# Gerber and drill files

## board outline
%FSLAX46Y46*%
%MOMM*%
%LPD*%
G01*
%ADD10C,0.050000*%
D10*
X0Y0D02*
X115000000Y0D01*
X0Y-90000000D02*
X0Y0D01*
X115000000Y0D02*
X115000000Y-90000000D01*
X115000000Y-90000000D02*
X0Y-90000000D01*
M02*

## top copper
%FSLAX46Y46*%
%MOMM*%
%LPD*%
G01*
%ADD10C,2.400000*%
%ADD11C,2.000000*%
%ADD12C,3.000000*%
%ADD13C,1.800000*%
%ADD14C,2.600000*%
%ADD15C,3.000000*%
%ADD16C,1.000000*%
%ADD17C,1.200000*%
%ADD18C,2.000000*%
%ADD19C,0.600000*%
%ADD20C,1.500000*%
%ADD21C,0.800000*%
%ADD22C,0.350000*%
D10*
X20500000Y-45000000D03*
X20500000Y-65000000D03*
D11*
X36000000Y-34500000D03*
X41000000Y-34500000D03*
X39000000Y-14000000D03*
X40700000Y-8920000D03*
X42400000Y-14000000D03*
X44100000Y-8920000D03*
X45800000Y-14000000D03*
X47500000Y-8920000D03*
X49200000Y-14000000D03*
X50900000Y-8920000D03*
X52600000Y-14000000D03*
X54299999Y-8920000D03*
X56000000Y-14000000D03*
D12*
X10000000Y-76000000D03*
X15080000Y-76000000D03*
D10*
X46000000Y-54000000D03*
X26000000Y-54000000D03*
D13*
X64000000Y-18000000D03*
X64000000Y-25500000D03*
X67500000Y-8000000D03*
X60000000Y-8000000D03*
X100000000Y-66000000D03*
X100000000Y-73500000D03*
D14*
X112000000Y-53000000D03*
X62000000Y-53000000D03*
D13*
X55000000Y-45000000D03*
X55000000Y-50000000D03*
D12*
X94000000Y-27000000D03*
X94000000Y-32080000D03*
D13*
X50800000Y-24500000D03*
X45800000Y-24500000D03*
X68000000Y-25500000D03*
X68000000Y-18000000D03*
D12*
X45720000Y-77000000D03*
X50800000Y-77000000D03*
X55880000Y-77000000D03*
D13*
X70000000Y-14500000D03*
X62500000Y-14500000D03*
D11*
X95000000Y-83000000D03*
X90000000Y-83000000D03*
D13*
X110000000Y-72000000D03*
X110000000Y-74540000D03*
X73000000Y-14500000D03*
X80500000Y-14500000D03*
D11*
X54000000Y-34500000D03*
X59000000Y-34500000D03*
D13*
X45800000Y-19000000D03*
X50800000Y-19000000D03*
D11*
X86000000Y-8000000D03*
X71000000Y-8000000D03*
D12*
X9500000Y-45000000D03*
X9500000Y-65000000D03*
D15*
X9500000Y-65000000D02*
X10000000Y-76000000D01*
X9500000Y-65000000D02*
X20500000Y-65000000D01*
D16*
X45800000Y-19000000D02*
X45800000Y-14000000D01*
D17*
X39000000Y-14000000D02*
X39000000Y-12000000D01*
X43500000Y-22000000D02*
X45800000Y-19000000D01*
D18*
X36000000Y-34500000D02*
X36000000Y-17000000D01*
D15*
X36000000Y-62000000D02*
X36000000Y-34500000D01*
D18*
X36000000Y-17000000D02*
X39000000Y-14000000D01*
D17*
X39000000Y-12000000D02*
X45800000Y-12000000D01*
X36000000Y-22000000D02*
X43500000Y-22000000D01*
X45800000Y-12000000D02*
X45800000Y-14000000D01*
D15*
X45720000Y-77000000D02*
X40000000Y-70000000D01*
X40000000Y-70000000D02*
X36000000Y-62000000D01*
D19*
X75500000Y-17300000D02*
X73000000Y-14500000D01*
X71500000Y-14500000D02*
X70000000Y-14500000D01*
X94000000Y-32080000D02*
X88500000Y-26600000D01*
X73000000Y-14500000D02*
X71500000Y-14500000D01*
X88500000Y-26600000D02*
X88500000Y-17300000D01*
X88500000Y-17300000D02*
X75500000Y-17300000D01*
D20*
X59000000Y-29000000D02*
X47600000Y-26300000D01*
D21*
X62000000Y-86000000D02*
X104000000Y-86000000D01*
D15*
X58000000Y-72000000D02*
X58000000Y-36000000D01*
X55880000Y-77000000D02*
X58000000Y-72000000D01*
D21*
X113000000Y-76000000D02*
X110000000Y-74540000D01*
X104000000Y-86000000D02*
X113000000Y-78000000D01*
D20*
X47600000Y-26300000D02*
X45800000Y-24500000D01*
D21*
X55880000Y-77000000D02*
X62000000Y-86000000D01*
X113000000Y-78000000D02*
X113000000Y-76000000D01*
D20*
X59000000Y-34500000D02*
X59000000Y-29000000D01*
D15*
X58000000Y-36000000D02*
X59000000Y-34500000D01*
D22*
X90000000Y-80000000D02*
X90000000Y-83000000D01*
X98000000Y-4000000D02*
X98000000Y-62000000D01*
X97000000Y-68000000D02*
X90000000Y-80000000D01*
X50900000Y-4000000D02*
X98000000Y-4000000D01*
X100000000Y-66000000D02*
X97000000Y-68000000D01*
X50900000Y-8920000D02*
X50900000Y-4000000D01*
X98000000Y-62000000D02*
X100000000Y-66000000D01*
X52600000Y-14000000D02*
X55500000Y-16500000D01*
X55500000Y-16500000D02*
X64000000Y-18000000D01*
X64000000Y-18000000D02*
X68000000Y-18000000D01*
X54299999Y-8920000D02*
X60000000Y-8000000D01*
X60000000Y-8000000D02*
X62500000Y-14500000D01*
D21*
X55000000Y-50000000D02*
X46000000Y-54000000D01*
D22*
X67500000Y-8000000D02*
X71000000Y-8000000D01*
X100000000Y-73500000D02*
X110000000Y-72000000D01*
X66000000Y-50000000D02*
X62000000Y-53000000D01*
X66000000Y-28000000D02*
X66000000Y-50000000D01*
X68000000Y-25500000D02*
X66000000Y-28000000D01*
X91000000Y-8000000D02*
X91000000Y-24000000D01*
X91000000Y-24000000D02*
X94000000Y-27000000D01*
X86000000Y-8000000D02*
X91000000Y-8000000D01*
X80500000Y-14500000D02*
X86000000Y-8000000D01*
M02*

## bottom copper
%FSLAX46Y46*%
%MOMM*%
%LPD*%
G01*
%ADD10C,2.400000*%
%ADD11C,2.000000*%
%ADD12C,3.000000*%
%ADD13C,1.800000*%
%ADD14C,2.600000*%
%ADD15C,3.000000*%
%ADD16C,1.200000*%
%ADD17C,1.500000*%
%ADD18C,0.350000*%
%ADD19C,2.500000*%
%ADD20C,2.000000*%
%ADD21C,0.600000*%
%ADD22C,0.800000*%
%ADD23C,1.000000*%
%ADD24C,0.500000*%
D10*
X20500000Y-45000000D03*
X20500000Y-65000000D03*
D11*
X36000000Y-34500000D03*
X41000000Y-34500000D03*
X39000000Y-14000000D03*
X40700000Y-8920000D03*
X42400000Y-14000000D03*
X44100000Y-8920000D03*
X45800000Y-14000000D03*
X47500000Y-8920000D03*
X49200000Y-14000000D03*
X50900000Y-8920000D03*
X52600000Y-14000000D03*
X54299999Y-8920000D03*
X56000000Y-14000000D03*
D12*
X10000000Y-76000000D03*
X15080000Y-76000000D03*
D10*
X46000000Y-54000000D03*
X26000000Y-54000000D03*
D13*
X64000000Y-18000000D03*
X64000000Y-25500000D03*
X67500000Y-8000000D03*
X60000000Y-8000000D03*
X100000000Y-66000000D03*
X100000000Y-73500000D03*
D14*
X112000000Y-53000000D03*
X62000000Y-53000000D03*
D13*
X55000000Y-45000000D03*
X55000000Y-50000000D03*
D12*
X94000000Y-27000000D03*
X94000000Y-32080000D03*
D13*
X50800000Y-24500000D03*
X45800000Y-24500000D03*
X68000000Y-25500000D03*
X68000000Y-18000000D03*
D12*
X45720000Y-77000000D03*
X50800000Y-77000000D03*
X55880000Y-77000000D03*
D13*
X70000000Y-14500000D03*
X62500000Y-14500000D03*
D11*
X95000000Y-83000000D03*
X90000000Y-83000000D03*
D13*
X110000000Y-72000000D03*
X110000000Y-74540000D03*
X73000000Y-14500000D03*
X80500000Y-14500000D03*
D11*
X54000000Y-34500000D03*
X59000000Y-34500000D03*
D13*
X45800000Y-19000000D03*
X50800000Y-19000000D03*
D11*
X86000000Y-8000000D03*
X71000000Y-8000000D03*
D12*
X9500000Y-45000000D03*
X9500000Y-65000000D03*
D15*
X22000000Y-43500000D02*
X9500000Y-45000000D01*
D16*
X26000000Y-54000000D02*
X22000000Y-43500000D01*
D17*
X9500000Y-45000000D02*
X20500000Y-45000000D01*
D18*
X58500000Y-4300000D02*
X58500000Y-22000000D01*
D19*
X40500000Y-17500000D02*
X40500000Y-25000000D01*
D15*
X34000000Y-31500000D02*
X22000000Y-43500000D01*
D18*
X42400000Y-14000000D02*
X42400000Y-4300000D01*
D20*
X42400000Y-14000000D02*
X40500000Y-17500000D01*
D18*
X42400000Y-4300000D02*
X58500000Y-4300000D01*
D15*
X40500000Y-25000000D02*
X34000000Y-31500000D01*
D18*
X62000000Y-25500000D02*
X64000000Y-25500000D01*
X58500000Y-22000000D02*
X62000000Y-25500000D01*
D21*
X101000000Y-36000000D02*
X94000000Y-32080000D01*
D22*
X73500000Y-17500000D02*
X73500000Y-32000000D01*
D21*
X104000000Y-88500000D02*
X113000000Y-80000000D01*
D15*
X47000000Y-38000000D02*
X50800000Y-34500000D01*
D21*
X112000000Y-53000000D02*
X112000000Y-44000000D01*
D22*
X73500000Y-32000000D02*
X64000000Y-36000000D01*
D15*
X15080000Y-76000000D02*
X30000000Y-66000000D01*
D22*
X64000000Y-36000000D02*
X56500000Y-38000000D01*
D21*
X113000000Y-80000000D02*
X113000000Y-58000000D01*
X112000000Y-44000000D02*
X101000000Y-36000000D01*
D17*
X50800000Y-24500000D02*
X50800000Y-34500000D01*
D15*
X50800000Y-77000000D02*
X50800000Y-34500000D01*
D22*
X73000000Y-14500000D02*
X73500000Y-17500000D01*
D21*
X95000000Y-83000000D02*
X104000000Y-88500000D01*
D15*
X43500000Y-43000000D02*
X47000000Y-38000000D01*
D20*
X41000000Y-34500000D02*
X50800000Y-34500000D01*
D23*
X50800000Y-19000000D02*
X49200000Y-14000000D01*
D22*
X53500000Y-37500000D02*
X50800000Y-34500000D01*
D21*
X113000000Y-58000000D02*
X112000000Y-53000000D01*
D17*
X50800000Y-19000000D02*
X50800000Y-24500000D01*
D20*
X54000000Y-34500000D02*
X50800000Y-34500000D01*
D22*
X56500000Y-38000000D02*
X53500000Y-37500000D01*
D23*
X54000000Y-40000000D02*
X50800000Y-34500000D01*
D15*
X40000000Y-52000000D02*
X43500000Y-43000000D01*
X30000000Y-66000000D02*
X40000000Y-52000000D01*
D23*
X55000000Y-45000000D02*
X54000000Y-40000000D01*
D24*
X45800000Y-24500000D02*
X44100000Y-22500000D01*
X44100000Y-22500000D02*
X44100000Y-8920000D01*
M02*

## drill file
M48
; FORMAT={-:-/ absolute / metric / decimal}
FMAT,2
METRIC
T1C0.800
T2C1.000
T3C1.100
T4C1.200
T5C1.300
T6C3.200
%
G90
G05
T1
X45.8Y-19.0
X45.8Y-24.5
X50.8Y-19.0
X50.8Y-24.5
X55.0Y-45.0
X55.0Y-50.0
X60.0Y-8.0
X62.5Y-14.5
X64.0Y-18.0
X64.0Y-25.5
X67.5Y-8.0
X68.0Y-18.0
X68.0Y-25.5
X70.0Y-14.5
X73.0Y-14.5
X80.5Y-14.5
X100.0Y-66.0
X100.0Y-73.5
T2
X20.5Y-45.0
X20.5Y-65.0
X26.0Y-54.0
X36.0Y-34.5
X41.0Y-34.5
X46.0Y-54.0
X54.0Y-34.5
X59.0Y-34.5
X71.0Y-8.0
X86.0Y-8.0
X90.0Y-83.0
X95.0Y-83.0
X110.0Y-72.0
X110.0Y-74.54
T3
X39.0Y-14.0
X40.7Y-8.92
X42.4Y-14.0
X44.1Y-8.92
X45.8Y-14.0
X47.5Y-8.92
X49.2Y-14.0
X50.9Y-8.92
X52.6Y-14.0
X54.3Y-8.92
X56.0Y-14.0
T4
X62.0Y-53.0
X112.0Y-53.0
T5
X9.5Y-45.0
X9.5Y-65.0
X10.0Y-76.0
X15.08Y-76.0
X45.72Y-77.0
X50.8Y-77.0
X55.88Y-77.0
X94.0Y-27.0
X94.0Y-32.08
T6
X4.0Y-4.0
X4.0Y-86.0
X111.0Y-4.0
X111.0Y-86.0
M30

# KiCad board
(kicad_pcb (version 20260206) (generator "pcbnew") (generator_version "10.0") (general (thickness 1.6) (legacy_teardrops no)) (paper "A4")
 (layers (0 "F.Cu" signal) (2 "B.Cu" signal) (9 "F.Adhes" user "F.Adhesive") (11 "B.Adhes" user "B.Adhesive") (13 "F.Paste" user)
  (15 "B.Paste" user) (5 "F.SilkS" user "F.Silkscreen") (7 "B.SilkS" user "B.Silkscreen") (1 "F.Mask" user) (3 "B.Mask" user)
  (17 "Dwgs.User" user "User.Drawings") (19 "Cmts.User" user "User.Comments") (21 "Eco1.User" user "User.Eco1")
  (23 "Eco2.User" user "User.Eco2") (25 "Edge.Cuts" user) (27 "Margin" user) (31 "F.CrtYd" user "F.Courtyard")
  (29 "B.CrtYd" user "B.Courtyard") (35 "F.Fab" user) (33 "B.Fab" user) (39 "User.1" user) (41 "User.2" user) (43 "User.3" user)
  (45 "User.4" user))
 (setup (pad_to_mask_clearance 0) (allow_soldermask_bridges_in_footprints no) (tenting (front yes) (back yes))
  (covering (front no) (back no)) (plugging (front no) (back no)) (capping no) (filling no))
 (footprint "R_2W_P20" (layer "F.Cu") (at 20.5 45 -90)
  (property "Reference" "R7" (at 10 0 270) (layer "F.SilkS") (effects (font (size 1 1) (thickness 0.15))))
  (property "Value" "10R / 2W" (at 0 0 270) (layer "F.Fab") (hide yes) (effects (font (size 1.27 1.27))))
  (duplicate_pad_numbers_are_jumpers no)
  (pad "1" thru_hole circle (at 0 0 270) (size 2.4 2.4) (drill 1) (layers "*.Cu" "*.Mask") (remove_unused_layers no) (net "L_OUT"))
  (pad "2" thru_hole circle (at 20 0 270) (size 2.4 2.4) (drill 1) (layers "*.Cu" "*.Mask") (remove_unused_layers no) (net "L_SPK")))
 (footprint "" (layer "F.Cu") (at 111 4)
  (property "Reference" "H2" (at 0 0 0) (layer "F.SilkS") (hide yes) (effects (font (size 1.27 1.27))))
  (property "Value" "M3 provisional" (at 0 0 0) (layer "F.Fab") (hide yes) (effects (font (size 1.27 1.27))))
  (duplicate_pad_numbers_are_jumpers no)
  (pad "" np_thru_hole circle (at 0 0) (size 3.2 3.2) (drill 3.2) (layers "*.Cu" "*.Mask")))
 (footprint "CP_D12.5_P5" (layer "F.Cu") (at 36 34.5)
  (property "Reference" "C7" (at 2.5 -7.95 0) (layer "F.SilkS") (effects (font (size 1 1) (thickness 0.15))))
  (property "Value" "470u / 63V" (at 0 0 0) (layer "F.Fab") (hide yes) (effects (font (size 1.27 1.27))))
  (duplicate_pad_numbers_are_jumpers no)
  (pad "1" thru_hole circle (at 0 0) (size 2 2) (drill 1) (layers "*.Cu" "*.Mask") (remove_unused_layers no) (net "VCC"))
  (pad "2" thru_hole circle (at 5 0) (size 2 2) (drill 1) (layers "*.Cu" "*.Mask") (remove_unused_layers no) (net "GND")))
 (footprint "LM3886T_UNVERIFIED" (layer "F.Cu") (at 39 14)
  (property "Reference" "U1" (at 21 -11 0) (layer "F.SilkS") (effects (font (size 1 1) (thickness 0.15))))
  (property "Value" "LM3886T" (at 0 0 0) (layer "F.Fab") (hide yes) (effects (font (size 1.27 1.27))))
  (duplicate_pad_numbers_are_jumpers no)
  (pad "1" thru_hole circle (at 0 0) (size 2 2) (drill 1.1) (layers "*.Cu" "*.Mask") (remove_unused_layers no) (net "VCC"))
  (pad "2" thru_hole circle (at 1.7 -5.08) (size 2 2) (drill 1.1) (layers "*.Cu" "*.Mask") (remove_unused_layers no)
   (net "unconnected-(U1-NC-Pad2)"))
  (pad "3" thru_hole circle (at 3.4 0) (size 2 2) (drill 1.1) (layers "*.Cu" "*.Mask") (remove_unused_layers no) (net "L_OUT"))
  (pad "4" thru_hole circle (at 5.1 -5.08) (size 2 2) (drill 1.1) (layers "*.Cu" "*.Mask") (remove_unused_layers no) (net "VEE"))
  (pad "5" thru_hole circle (at 6.8 0) (size 2 2) (drill 1.1) (layers "*.Cu" "*.Mask") (remove_unused_layers no) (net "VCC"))
  (pad "6" thru_hole circle (at 8.5 -5.08) (size 2 2) (drill 1.1) (layers "*.Cu" "*.Mask") (remove_unused_layers no)
   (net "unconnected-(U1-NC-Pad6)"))
  (pad "7" thru_hole circle (at 10.2 0) (size 2 2) (drill 1.1) (layers "*.Cu" "*.Mask") (remove_unused_layers no) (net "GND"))
  (pad "8" thru_hole circle (at 11.9 -5.08) (size 2 2) (drill 1.1) (layers "*.Cu" "*.Mask") (remove_unused_layers no) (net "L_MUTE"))
  (pad "9" thru_hole circle (at 13.6 0) (size 2 2) (drill 1.1) (layers "*.Cu" "*.Mask") (remove_unused_layers no) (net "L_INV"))
  (pad "10" thru_hole circle (at 15.299999 -5.08) (size 2 2) (drill 1.1) (layers "*.Cu" "*.Mask") (remove_unused_layers no) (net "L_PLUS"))
  (pad "11" thru_hole circle (at 17 0) (size 2 2) (drill 1.1) (layers "*.Cu" "*.Mask") (remove_unused_layers no)
   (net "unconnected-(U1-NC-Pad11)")))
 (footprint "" (layer "F.Cu") (at 4 4)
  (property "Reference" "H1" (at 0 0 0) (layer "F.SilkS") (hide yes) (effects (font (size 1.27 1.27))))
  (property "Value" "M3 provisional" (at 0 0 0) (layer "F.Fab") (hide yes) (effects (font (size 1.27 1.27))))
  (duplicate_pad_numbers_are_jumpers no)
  (pad "" np_thru_hole circle (at 0 0) (size 3.2 3.2) (drill 3.2) (layers "*.Cu" "*.Mask")))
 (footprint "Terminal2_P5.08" (layer "F.Cu") (at 10 76)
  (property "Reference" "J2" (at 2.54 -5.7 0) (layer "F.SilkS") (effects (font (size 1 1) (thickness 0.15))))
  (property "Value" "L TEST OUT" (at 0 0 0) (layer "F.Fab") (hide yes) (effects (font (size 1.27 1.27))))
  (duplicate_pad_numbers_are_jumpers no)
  (pad "1" thru_hole circle (at 0 0) (size 3 3) (drill 1.3) (layers "*.Cu" "*.Mask") (remove_unused_layers no) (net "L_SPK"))
  (pad "2" thru_hole circle (at 5.08 0) (size 3 3) (drill 1.3) (layers "*.Cu" "*.Mask") (remove_unused_layers no) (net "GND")))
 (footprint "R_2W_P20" (layer "F.Cu") (at 46 54 180)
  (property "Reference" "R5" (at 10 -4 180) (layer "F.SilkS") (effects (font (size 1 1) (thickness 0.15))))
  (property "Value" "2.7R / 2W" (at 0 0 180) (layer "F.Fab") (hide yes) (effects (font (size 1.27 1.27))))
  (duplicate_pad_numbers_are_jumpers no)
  (pad "1" thru_hole circle (at 0 0 180) (size 2.4 2.4) (drill 1) (layers "*.Cu" "*.Mask") (remove_unused_layers no) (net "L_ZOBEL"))
  (pad "2" thru_hole circle (at 20 0 180) (size 2.4 2.4) (drill 1) (layers "*.Cu" "*.Mask") (remove_unused_layers no) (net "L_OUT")))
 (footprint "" (layer "F.Cu") (at 4 86)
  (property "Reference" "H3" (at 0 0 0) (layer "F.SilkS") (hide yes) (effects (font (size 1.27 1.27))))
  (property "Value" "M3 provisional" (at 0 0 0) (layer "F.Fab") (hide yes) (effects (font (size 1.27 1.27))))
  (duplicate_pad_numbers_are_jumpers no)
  (pad "" np_thru_hole circle (at 0 0) (size 3.2 3.2) (drill 3.2) (layers "*.Cu" "*.Mask")))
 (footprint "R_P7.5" (layer "F.Cu") (at 64 18 -90)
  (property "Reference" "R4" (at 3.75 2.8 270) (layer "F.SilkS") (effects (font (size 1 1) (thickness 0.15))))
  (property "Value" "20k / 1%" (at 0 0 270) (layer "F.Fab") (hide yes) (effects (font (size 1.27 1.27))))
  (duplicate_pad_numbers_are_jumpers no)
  (pad "1" thru_hole circle (at 0 0 270) (size 1.8 1.8) (drill 0.8) (layers "*.Cu" "*.Mask") (remove_unused_layers no) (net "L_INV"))
  (pad "2" thru_hole circle (at 7.5 0 270) (size 1.8 1.8) (drill 0.8) (layers "*.Cu" "*.Mask") (remove_unused_layers no) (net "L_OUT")))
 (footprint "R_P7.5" (layer "F.Cu") (at 67.5 8 180)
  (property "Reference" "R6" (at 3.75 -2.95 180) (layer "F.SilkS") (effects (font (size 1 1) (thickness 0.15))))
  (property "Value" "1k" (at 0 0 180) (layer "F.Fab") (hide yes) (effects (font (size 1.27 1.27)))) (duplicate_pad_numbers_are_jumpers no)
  (pad "1" thru_hole circle (at 0 0 180) (size 1.8 1.8) (drill 0.8) (layers "*.Cu" "*.Mask") (remove_unused_layers no) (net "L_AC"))
  (pad "2" thru_hole circle (at 7.5 0 180) (size 1.8 1.8) (drill 0.8) (layers "*.Cu" "*.Mask") (remove_unused_layers no) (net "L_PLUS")))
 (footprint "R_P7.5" (layer "F.Cu") (at 100 66 -90)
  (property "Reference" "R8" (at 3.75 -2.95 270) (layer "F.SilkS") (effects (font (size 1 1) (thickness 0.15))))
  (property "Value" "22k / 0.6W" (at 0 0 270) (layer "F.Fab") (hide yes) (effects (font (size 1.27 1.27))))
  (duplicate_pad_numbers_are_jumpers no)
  (pad "1" thru_hole circle (at 0 0 270) (size 1.8 1.8) (drill 0.8) (layers "*.Cu" "*.Mask") (remove_unused_layers no) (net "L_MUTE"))
  (pad "2" thru_hole circle (at 7.5 0 270) (size 1.8 1.8) (drill 0.8) (layers "*.Cu" "*.Mask") (remove_unused_layers no) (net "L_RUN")))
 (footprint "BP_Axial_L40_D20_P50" (layer "F.Cu") (at 112 53 180)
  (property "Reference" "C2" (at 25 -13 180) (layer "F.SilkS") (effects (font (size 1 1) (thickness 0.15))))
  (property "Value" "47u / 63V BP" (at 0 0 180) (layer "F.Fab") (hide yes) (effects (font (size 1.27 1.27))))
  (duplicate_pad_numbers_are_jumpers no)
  (pad "1" thru_hole circle (at 0 0 180) (size 2.6 2.6) (drill 1.2) (layers "*.Cu" "*.Mask") (remove_unused_layers no) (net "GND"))
  (pad "2" thru_hole circle (at 50 0 180) (size 2.6 2.6) (drill 1.2) (layers "*.Cu" "*.Mask") (remove_unused_layers no) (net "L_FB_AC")))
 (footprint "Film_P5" (layer "F.Cu") (at 55 45 -90)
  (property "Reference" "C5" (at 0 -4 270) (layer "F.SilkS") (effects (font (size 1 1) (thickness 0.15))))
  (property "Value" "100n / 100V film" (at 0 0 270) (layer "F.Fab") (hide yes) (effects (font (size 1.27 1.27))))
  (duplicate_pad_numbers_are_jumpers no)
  (pad "1" thru_hole circle (at 0 0 270) (size 1.8 1.8) (drill 0.8) (layers "*.Cu" "*.Mask") (remove_unused_layers no) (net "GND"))
  (pad "2" thru_hole circle (at 5 0 270) (size 1.8 1.8) (drill 0.8) (layers "*.Cu" "*.Mask") (remove_unused_layers no) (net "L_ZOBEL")))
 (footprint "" (layer "F.Cu") (at 111 86)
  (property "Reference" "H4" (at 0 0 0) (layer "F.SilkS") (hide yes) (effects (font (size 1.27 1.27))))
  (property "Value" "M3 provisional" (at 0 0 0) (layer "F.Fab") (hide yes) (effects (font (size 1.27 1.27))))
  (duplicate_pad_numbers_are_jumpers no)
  (pad "" np_thru_hole circle (at 0 0) (size 3.2 3.2) (drill 3.2) (layers "*.Cu" "*.Mask")))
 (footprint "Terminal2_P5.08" (layer "F.Cu") (at 94 27 -90)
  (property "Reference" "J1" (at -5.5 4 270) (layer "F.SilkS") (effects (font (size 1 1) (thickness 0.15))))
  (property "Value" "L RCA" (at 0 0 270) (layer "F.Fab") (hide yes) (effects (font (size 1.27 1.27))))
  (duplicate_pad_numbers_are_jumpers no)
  (pad "1" thru_hole circle (at 0 0 270) (size 3 3) (drill 1.3) (layers "*.Cu" "*.Mask") (remove_unused_layers no) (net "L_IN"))
  (pad "2" thru_hole circle (at 5.08 0 270) (size 3 3) (drill 1.3) (layers "*.Cu" "*.Mask") (remove_unused_layers no) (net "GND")))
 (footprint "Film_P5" (layer "F.Cu") (at 50.8 24.5 180)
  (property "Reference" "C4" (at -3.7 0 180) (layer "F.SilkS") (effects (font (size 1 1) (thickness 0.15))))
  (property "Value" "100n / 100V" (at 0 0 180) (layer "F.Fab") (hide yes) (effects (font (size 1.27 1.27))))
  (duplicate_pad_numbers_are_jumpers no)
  (pad "1" thru_hole circle (at 0 0 180) (size 1.8 1.8) (drill 0.8) (layers "*.Cu" "*.Mask") (remove_unused_layers no) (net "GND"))
  (pad "2" thru_hole circle (at 5 0 180) (size 1.8 1.8) (drill 0.8) (layers "*.Cu" "*.Mask") (remove_unused_layers no) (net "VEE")))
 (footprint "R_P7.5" (layer "F.Cu") (at 68 25.5 90)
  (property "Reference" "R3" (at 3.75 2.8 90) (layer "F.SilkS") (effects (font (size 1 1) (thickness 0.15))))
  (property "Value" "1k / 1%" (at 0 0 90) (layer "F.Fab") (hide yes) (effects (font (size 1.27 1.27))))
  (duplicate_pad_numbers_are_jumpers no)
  (pad "1" thru_hole circle (at 0 0 90) (size 1.8 1.8) (drill 0.8) (layers "*.Cu" "*.Mask") (remove_unused_layers no) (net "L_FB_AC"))
  (pad "2" thru_hole circle (at 7.5 0 90) (size 1.8 1.8) (drill 0.8) (layers "*.Cu" "*.Mask") (remove_unused_layers no) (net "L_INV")))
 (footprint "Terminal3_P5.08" (layer "F.Cu") (at 45.72 77)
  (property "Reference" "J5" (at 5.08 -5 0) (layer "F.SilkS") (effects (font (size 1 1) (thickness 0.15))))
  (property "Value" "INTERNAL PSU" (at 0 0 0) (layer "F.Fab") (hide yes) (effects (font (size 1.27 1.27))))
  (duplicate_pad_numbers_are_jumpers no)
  (pad "1" thru_hole circle (at 0 0) (size 3 3) (drill 1.3) (layers "*.Cu" "*.Mask") (remove_unused_layers no) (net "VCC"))
  (pad "2" thru_hole circle (at 5.08 0) (size 3 3) (drill 1.3) (layers "*.Cu" "*.Mask") (remove_unused_layers no) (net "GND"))
  (pad "3" thru_hole circle (at 10.16 0) (size 3 3) (drill 1.3) (layers "*.Cu" "*.Mask") (remove_unused_layers no) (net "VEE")))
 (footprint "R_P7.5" (layer "F.Cu") (at 70 14.5 180)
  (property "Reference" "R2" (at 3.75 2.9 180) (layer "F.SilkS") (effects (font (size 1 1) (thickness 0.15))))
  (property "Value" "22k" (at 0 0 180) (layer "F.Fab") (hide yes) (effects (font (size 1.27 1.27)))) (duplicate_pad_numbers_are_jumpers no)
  (pad "1" thru_hole circle (at 0 0 180) (size 1.8 1.8) (drill 0.8) (layers "*.Cu" "*.Mask") (remove_unused_layers no) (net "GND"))
  (pad "2" thru_hole circle (at 7.5 0 180) (size 1.8 1.8) (drill 0.8) (layers "*.Cu" "*.Mask") (remove_unused_layers no) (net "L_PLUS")))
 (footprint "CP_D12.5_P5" (layer "F.Cu") (at 95 83 180)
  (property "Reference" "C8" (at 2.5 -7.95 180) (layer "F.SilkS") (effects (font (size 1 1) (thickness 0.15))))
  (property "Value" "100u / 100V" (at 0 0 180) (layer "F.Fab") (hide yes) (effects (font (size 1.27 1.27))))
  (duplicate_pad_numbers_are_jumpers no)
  (pad "1" thru_hole circle (at 0 0 180) (size 2 2) (drill 1) (layers "*.Cu" "*.Mask") (remove_unused_layers no) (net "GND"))
  (pad "2" thru_hole circle (at 5 0 180) (size 2 2) (drill 1) (layers "*.Cu" "*.Mask") (remove_unused_layers no) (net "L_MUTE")))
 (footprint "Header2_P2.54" (layer "F.Cu") (at 110 72 -90)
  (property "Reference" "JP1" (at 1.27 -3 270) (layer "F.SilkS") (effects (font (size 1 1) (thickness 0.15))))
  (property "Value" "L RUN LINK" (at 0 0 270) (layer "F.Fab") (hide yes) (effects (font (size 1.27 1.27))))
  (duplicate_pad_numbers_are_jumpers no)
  (pad "1" thru_hole circle (at 0 0 270) (size 1.8 1.8) (drill 1) (layers "*.Cu" "*.Mask") (remove_unused_layers no) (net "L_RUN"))
  (pad "2" thru_hole circle (at 2.54 0 270) (size 1.8 1.8) (drill 1) (layers "*.Cu" "*.Mask") (remove_unused_layers no) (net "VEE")))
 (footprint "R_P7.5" (layer "F.Cu") (at 73 14.5)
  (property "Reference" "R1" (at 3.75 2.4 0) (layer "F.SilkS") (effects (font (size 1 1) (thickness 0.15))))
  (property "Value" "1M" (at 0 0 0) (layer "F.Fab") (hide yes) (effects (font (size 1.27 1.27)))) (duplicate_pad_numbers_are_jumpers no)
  (pad "1" thru_hole circle (at 0 0) (size 1.8 1.8) (drill 0.8) (layers "*.Cu" "*.Mask") (remove_unused_layers no) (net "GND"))
  (pad "2" thru_hole circle (at 7.5 0) (size 1.8 1.8) (drill 0.8) (layers "*.Cu" "*.Mask") (remove_unused_layers no) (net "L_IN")))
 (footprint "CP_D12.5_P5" (layer "F.Cu") (at 54 34.5)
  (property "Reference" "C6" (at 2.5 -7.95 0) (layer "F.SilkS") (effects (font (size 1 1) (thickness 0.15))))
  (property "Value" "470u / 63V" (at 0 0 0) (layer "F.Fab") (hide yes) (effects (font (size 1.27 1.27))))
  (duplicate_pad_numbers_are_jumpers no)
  (pad "1" thru_hole circle (at 0 0) (size 2 2) (drill 1) (layers "*.Cu" "*.Mask") (remove_unused_layers no) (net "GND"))
  (pad "2" thru_hole circle (at 5 0) (size 2 2) (drill 1) (layers "*.Cu" "*.Mask") (remove_unused_layers no) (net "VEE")))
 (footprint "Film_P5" (layer "F.Cu") (at 45.8 19)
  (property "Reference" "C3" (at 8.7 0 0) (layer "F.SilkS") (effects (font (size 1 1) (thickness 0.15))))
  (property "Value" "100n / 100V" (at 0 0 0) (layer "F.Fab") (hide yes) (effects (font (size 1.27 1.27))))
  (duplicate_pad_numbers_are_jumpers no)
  (pad "1" thru_hole circle (at 0 0) (size 1.8 1.8) (drill 0.8) (layers "*.Cu" "*.Mask") (remove_unused_layers no) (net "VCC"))
  (pad "2" thru_hole circle (at 5 0) (size 1.8 1.8) (drill 0.8) (layers "*.Cu" "*.Mask") (remove_unused_layers no) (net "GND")))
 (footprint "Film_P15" (layer "F.Cu") (at 86 8 180)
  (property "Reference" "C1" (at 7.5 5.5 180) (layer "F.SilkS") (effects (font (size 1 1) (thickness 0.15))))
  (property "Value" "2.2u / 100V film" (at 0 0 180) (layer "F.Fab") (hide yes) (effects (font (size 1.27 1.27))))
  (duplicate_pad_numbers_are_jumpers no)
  (pad "1" thru_hole circle (at 0 0 180) (size 2 2) (drill 1) (layers "*.Cu" "*.Mask") (remove_unused_layers no) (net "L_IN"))
  (pad "2" thru_hole circle (at 15 0 180) (size 2 2) (drill 1) (layers "*.Cu" "*.Mask") (remove_unused_layers no) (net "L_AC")))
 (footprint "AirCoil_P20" (layer "F.Cu") (at 9.5 45 -90)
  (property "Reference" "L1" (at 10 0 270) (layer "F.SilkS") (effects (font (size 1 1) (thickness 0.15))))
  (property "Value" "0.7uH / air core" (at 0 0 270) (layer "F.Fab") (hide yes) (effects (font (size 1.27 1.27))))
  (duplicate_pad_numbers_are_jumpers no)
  (pad "1" thru_hole circle (at 0 0 270) (size 3 3) (drill 1.3) (layers "*.Cu" "*.Mask") (remove_unused_layers no) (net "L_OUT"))
  (pad "2" thru_hole circle (at 20 0 270) (size 3 3) (drill 1.3) (layers "*.Cu" "*.Mask") (remove_unused_layers no) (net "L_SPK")))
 (gr_line (start 0 0) (end 115 0) (stroke (width 0.05) (type default)) (layer "Edge.Cuts"))
 (gr_line (start 0 90) (end 0 0) (stroke (width 0.05) (type default)) (layer "Edge.Cuts"))
 (gr_line (start 115 0) (end 115 90) (stroke (width 0.05) (type default)) (layer "Edge.Cuts"))
 (gr_line (start 115 90) (end 0 90) (stroke (width 0.05) (type default)) (layer "Edge.Cuts"))
 (segment (start 22 43.5) (end 9.5 45) (width 3) (layer "B.Cu") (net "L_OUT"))
 (segment (start 26 54) (end 22 43.5) (width 1.2) (layer "B.Cu") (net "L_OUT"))
 (segment (start 9.5 45) (end 20.5 45) (width 1.5) (layer "B.Cu") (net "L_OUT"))
 (segment (start 58.5 4.3) (end 58.5 22) (width 0.35) (layer "B.Cu") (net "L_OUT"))
 (segment (start 40.5 17.5) (end 40.5 25) (width 2.5) (layer "B.Cu") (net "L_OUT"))
 (segment (start 34 31.5) (end 22 43.5) (width 3) (layer "B.Cu") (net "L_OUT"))
 (segment (start 42.4 14) (end 42.4 4.3) (width 0.35) (layer "B.Cu") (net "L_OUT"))
 (segment (start 42.4 14) (end 40.5 17.5) (width 2) (layer "B.Cu") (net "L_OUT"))
 (segment (start 42.4 4.3) (end 58.5 4.3) (width 0.35) (layer "B.Cu") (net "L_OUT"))
 (segment (start 40.5 25) (end 34 31.5) (width 3) (layer "B.Cu") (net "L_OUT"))
 (segment (start 62 25.5) (end 64 25.5) (width 0.35) (layer "B.Cu") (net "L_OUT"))
 (segment (start 58.5 22) (end 62 25.5) (width 0.35) (layer "B.Cu") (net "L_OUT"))
 (segment (start 9.5 65) (end 10 76) (width 3) (layer "F.Cu") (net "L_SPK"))
 (segment (start 9.5 65) (end 20.5 65) (width 3) (layer "F.Cu") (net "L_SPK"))
 (segment (start 45.8 19) (end 45.8 14) (width 1) (layer "F.Cu") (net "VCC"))
 (segment (start 39 14) (end 39 12) (width 1.2) (layer "F.Cu") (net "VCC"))
 (segment (start 43.5 22) (end 45.8 19) (width 1.2) (layer "F.Cu") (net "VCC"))
 (segment (start 36 34.5) (end 36 17) (width 2) (layer "F.Cu") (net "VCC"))
 (segment (start 36 62) (end 36 34.5) (width 3) (layer "F.Cu") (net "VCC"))
 (segment (start 36 17) (end 39 14) (width 2) (layer "F.Cu") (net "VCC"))
 (segment (start 39 12) (end 45.8 12) (width 1.2) (layer "F.Cu") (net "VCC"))
 (segment (start 36 22) (end 43.5 22) (width 1.2) (layer "F.Cu") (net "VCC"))
 (segment (start 45.8 12) (end 45.8 14) (width 1.2) (layer "F.Cu") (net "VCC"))
 (segment (start 45.72 77) (end 40 70) (width 3) (layer "F.Cu") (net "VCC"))
 (segment (start 40 70) (end 36 62) (width 3) (layer "F.Cu") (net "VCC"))
 (segment (start 75.5 17.3) (end 73 14.5) (width 0.6) (layer "F.Cu") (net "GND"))
 (segment (start 71.5 14.5) (end 70 14.5) (width 0.6) (layer "F.Cu") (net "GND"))
 (segment (start 94 32.08) (end 88.5 26.6) (width 0.6) (layer "F.Cu") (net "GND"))
 (segment (start 73 14.5) (end 71.5 14.5) (width 0.6) (layer "F.Cu") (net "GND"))
 (segment (start 88.5 26.6) (end 88.5 17.3) (width 0.6) (layer "F.Cu") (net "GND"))
 (segment (start 88.5 17.3) (end 75.5 17.3) (width 0.6) (layer "F.Cu") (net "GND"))
 (segment (start 101 36) (end 94 32.08) (width 0.6) (layer "B.Cu") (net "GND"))
 (segment (start 73.5 17.5) (end 73.5 32) (width 0.8) (layer "B.Cu") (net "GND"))
 (segment (start 104 88.5) (end 113 80) (width 0.6) (layer "B.Cu") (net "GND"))
 (segment (start 47 38) (end 50.8 34.5) (width 3) (layer "B.Cu") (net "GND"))
 (segment (start 112 53) (end 112 44) (width 0.6) (layer "B.Cu") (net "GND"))
 (segment (start 73.5 32) (end 64 36) (width 0.8) (layer "B.Cu") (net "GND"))
 (segment (start 15.08 76) (end 30 66) (width 3) (layer "B.Cu") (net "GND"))
 (segment (start 64 36) (end 56.5 38) (width 0.8) (layer "B.Cu") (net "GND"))
 (segment (start 113 80) (end 113 58) (width 0.6) (layer "B.Cu") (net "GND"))
 (segment (start 112 44) (end 101 36) (width 0.6) (layer "B.Cu") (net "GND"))
 (segment (start 50.8 24.5) (end 50.8 34.5) (width 1.5) (layer "B.Cu") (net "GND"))
 (segment (start 50.8 77) (end 50.8 34.5) (width 3) (layer "B.Cu") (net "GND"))
 (segment (start 73 14.5) (end 73.5 17.5) (width 0.8) (layer "B.Cu") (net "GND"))
 (segment (start 95 83) (end 104 88.5) (width 0.6) (layer "B.Cu") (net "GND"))
 (segment (start 43.5 43) (end 47 38) (width 3) (layer "B.Cu") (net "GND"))
 (segment (start 41 34.5) (end 50.8 34.5) (width 2) (layer "B.Cu") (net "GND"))
 (segment (start 50.8 19) (end 49.2 14) (width 1) (layer "B.Cu") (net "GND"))
 (segment (start 53.5 37.5) (end 50.8 34.5) (width 0.8) (layer "B.Cu") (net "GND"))
 (segment (start 113 58) (end 112 53) (width 0.6) (layer "B.Cu") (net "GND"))
 (segment (start 50.8 19) (end 50.8 24.5) (width 1.5) (layer "B.Cu") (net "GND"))
 (segment (start 54 34.5) (end 50.8 34.5) (width 2) (layer "B.Cu") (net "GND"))
 (segment (start 56.5 38) (end 53.5 37.5) (width 0.8) (layer "B.Cu") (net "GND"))
 (segment (start 54 40) (end 50.8 34.5) (width 1) (layer "B.Cu") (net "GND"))
 (segment (start 40 52) (end 43.5 43) (width 3) (layer "B.Cu") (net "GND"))
 (segment (start 30 66) (end 40 52) (width 3) (layer "B.Cu") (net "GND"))
 (segment (start 55 45) (end 54 40) (width 1) (layer "B.Cu") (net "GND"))
 (segment (start 59 29) (end 47.6 26.3) (width 1.5) (layer "F.Cu") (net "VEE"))
 (segment (start 62 86) (end 104 86) (width 0.8) (layer "F.Cu") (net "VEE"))
 (segment (start 58 72) (end 58 36) (width 3) (layer "F.Cu") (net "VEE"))
 (segment (start 55.88 77) (end 58 72) (width 3) (layer "F.Cu") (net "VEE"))
 (segment (start 113 76) (end 110 74.54) (width 0.8) (layer "F.Cu") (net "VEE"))
 (segment (start 104 86) (end 113 78) (width 0.8) (layer "F.Cu") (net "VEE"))
 (segment (start 47.6 26.3) (end 45.8 24.5) (width 1.5) (layer "F.Cu") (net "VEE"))
 (segment (start 55.88 77) (end 62 86) (width 0.8) (layer "F.Cu") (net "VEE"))
 (segment (start 113 78) (end 113 76) (width 0.8) (layer "F.Cu") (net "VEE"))
 (segment (start 59 34.5) (end 59 29) (width 1.5) (layer "F.Cu") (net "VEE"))
 (segment (start 58 36) (end 59 34.5) (width 3) (layer "F.Cu") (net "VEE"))
 (segment (start 45.8 24.5) (end 44.1 22.5) (width 0.5) (layer "B.Cu") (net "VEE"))
 (segment (start 44.1 22.5) (end 44.1 8.92) (width 0.5) (layer "B.Cu") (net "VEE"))
 (segment (start 90 80) (end 90 83) (width 0.35) (layer "F.Cu") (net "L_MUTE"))
 (segment (start 98 4) (end 98 62) (width 0.35) (layer "F.Cu") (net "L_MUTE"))
 (segment (start 97 68) (end 90 80) (width 0.35) (layer "F.Cu") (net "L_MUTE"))
 (segment (start 50.9 4) (end 98 4) (width 0.35) (layer "F.Cu") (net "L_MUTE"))
 (segment (start 100 66) (end 97 68) (width 0.35) (layer "F.Cu") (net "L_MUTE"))
 (segment (start 50.9 8.92) (end 50.9 4) (width 0.35) (layer "F.Cu") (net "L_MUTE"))
 (segment (start 98 62) (end 100 66) (width 0.35) (layer "F.Cu") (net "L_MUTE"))
 (segment (start 52.6 14) (end 55.5 16.5) (width 0.35) (layer "F.Cu") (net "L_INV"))
 (segment (start 55.5 16.5) (end 64 18) (width 0.35) (layer "F.Cu") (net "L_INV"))
 (segment (start 64 18) (end 68 18) (width 0.35) (layer "F.Cu") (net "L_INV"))
 (segment (start 54.299999 8.92) (end 60 8) (width 0.35) (layer "F.Cu") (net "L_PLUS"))
 (segment (start 60 8) (end 62.5 14.5) (width 0.35) (layer "F.Cu") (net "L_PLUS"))
 (segment (start 55 50) (end 46 54) (width 0.8) (layer "F.Cu") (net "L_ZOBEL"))
 (segment (start 67.5 8) (end 71 8) (width 0.35) (layer "F.Cu") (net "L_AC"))
 (segment (start 100 73.5) (end 110 72) (width 0.35) (layer "F.Cu") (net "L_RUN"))
 (segment (start 66 50) (end 62 53) (width 0.35) (layer "F.Cu") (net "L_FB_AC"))
 (segment (start 66 28) (end 66 50) (width 0.35) (layer "F.Cu") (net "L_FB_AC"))
 (segment (start 68 25.5) (end 66 28) (width 0.35) (layer "F.Cu") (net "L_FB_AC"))
 (segment (start 91 8) (end 91 24) (width 0.35) (layer "F.Cu") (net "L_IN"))
 (segment (start 91 24) (end 94 27) (width 0.35) (layer "F.Cu") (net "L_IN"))
 (segment (start 86 8) (end 91 8) (width 0.35) (layer "F.Cu") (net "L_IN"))
 (segment (start 80.5 14.5) (end 86 8) (width 0.35) (layer "F.Cu") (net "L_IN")))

